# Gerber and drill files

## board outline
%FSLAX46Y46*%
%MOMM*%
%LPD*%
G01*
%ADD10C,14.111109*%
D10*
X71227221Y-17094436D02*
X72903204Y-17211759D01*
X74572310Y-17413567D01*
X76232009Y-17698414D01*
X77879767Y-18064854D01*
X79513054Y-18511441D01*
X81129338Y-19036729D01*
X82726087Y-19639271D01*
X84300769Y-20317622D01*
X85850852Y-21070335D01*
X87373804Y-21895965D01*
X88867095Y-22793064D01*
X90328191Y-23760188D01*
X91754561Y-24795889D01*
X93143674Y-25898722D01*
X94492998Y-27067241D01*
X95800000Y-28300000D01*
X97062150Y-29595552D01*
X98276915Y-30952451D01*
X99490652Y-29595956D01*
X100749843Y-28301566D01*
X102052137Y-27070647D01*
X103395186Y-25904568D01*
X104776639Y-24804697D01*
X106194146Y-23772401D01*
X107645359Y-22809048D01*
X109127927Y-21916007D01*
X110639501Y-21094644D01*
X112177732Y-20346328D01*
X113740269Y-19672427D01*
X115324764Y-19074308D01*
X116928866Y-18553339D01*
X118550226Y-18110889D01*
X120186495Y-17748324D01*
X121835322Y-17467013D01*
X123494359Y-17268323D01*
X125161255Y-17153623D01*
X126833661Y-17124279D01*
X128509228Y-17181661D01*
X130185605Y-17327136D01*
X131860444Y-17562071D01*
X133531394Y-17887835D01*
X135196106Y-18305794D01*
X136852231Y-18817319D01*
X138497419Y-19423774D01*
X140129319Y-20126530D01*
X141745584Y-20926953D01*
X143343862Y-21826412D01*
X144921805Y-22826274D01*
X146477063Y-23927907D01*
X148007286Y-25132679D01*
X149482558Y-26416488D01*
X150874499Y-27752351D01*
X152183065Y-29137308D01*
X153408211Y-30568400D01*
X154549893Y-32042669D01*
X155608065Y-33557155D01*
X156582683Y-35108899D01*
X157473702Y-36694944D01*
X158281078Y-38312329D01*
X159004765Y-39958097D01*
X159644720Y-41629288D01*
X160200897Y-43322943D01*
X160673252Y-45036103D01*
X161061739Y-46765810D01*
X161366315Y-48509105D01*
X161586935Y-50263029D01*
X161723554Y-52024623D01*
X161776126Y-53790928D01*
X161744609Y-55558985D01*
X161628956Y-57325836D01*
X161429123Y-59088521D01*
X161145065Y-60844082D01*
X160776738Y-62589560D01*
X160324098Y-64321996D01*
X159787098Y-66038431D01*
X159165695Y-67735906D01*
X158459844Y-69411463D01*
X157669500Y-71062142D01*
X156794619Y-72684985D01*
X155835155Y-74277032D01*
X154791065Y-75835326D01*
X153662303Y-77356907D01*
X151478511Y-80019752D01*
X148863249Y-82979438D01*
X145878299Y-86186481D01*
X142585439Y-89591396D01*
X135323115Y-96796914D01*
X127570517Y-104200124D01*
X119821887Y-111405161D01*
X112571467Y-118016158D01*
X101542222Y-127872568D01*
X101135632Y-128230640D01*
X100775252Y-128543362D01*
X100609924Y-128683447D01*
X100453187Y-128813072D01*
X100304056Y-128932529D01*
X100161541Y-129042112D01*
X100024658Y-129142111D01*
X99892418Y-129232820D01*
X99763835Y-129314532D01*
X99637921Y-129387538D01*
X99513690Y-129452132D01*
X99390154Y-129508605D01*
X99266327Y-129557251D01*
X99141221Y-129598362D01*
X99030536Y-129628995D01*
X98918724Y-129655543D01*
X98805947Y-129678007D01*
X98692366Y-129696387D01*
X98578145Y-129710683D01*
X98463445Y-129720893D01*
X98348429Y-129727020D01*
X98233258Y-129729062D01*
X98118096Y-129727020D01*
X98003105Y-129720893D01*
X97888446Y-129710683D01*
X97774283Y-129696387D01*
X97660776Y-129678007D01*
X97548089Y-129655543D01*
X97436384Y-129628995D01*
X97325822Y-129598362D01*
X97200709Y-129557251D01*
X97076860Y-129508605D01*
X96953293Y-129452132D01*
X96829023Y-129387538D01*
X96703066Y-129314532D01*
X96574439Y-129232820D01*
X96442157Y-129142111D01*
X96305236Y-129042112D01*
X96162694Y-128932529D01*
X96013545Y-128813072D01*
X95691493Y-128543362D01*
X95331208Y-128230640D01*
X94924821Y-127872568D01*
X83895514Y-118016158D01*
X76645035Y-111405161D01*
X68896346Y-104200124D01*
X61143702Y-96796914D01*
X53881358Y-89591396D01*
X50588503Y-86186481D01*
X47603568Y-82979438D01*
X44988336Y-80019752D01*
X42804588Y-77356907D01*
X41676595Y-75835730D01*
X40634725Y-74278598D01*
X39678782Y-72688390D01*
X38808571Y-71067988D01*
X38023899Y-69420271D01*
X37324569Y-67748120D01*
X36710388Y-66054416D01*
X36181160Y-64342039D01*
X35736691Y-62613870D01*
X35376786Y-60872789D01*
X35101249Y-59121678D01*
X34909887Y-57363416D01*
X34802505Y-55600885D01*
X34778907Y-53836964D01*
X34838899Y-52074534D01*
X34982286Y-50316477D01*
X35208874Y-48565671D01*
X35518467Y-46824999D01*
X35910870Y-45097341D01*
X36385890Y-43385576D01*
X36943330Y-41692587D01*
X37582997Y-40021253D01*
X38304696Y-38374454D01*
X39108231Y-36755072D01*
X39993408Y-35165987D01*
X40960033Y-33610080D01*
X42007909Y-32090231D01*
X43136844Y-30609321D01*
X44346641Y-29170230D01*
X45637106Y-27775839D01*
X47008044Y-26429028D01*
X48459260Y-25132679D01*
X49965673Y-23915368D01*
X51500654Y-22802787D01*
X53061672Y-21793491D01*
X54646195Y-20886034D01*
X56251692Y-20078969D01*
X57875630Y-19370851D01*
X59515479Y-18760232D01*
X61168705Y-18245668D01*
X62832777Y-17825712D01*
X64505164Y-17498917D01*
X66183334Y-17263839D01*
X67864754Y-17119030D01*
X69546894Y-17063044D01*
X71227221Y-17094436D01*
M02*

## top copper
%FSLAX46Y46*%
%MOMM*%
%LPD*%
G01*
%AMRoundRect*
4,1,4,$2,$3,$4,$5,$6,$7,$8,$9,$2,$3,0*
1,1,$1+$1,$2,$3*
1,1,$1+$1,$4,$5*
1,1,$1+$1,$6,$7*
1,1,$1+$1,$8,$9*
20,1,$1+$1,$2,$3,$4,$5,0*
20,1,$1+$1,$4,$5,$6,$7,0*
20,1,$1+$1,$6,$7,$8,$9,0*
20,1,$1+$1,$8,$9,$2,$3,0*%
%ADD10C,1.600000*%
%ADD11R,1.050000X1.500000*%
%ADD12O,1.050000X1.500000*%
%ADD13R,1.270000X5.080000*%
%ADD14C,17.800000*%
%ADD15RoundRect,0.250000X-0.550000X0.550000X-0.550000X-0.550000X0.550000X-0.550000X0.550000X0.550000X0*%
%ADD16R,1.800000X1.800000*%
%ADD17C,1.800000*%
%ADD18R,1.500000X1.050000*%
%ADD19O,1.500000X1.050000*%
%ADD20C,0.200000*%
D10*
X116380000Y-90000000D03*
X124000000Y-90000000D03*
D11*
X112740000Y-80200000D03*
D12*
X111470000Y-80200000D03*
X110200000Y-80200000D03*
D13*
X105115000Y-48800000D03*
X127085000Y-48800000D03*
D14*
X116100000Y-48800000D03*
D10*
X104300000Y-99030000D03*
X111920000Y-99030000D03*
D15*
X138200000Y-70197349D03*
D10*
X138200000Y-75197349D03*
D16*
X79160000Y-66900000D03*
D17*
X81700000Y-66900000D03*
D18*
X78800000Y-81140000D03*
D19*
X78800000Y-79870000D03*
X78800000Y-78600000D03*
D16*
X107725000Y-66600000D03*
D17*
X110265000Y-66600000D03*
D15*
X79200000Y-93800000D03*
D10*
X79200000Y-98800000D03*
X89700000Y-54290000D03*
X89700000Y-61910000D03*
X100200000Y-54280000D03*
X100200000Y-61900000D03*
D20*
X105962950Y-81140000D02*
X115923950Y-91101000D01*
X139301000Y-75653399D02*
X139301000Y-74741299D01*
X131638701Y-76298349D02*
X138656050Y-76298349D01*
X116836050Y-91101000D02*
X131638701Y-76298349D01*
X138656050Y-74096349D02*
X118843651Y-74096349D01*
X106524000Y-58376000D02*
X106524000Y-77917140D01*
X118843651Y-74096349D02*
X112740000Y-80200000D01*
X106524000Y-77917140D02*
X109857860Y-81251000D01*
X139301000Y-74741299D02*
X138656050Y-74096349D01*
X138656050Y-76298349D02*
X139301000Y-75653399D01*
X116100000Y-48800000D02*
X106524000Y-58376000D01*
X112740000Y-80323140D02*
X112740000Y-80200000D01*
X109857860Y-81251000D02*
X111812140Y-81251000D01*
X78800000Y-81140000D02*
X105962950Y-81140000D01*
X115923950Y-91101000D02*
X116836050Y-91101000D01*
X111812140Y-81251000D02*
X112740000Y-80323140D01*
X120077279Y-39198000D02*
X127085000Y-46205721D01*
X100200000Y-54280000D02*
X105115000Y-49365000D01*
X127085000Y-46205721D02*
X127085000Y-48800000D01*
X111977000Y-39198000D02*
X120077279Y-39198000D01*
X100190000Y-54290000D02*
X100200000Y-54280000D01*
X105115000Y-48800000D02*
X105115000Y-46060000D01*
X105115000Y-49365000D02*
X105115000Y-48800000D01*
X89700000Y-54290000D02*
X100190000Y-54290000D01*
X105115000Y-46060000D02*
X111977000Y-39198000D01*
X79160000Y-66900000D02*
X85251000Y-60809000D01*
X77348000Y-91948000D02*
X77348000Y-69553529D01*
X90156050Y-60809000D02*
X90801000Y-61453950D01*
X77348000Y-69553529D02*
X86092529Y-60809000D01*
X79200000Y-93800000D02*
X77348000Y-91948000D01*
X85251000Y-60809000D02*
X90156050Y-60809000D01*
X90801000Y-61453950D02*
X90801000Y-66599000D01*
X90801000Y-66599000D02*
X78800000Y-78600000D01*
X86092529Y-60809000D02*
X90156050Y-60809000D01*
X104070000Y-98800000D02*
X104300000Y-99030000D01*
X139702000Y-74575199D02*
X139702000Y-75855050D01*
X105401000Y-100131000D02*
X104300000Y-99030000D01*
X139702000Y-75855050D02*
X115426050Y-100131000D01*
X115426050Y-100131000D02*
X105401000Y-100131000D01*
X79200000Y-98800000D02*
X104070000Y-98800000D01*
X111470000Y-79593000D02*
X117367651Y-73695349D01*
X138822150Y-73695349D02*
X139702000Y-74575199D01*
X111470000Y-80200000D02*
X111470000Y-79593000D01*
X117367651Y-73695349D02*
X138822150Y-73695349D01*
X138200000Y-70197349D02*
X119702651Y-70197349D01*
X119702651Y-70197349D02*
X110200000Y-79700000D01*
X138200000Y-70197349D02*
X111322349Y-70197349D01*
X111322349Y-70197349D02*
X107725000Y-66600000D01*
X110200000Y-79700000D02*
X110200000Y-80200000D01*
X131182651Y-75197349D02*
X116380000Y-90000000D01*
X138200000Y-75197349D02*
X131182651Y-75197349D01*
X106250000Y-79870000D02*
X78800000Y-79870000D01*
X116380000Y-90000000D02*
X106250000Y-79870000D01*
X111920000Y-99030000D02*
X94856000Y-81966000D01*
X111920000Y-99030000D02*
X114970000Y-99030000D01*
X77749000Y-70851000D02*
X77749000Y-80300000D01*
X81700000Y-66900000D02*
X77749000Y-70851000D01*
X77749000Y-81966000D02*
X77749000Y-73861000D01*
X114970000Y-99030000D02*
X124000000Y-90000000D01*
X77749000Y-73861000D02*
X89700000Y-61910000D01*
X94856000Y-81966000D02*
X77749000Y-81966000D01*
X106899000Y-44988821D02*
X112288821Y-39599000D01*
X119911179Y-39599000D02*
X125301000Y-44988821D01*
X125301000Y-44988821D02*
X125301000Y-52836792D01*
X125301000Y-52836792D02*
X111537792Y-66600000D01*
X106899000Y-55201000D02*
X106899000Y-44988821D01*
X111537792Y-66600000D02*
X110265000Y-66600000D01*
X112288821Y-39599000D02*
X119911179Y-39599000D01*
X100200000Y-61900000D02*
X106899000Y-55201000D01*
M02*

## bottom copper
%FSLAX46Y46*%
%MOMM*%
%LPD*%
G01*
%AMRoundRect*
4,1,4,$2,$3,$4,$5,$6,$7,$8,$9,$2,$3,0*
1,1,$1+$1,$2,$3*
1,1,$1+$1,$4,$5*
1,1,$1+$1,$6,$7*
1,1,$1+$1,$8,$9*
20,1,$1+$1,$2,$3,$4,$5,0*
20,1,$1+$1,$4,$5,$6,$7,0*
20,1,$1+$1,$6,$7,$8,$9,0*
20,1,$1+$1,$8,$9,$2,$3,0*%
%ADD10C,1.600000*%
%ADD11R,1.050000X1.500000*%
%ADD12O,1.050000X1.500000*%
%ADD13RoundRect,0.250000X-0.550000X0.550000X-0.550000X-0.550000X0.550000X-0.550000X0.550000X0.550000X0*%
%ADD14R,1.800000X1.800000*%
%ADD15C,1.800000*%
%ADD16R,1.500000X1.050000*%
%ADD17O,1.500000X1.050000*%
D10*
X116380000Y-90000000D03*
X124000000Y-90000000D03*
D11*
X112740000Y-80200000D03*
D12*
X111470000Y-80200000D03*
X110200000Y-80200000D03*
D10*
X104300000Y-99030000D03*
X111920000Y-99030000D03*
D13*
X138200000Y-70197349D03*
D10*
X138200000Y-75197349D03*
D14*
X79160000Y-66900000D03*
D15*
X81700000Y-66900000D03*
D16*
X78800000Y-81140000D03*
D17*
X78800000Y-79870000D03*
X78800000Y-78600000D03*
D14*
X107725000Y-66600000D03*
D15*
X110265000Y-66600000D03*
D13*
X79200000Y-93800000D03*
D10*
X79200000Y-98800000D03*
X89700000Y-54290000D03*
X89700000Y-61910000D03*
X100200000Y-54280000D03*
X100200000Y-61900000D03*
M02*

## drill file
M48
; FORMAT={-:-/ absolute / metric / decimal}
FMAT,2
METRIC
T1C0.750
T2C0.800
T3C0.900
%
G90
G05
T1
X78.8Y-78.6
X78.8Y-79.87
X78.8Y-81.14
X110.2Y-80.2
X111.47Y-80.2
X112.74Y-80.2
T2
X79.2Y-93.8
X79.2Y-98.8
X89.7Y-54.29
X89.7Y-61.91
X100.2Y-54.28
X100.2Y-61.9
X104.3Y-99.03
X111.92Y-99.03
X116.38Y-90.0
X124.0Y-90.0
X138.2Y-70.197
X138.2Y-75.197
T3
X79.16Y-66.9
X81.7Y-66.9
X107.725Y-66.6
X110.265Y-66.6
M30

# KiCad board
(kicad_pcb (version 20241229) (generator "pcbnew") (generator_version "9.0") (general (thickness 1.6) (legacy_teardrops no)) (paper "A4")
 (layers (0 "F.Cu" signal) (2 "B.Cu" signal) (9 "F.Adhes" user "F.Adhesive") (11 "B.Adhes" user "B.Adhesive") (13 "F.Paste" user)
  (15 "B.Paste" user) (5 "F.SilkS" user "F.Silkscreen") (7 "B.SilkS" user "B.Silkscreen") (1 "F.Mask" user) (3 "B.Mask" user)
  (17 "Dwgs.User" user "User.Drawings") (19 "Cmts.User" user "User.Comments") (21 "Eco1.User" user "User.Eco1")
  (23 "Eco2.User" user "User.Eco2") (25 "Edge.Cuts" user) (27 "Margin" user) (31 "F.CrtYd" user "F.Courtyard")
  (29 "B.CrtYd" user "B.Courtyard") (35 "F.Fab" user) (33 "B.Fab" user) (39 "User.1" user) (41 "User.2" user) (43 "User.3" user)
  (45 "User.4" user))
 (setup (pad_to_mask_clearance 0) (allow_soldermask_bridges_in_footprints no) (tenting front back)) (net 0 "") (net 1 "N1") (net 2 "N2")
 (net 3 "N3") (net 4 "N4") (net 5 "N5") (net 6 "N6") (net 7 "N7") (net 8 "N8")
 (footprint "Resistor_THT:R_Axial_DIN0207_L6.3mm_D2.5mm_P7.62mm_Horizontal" (layer "F.Cu") (at 116.38 90)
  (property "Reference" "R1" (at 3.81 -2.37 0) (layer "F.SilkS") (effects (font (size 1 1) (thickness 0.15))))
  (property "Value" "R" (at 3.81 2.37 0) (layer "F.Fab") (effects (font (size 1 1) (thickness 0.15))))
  (pad "1" thru_hole circle (at 0 0) (size 1.6 1.6) (drill 0.8) (layers "*.Cu" "*.Mask") (remove_unused_layers no) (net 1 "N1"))
  (pad "2" thru_hole circle (at 7.62 0) (size 1.6 1.6) (drill 0.8) (layers "*.Cu" "*.Mask") (remove_unused_layers no) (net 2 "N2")))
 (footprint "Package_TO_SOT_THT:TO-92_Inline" (layer "F.Cu") (at 112.74 80.2 180)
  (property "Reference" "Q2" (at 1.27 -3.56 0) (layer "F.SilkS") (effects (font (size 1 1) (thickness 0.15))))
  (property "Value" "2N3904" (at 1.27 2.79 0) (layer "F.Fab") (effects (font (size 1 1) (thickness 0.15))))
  (pad "1" thru_hole rect (at 0 0 180) (size 1.05 1.5) (drill 0.75) (layers "*.Cu" "*.Mask") (remove_unused_layers no) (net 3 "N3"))
  (pad "2" thru_hole oval (at 1.27 0 180) (size 1.05 1.5) (drill 0.75) (layers "*.Cu" "*.Mask") (remove_unused_layers no) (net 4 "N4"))
  (pad "3" thru_hole oval (at 2.54 0 180) (size 1.05 1.5) (drill 0.75) (layers "*.Cu" "*.Mask") (remove_unused_layers no) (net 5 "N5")))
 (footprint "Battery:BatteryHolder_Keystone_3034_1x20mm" (layer "F.Cu") (at 116.1 48.8)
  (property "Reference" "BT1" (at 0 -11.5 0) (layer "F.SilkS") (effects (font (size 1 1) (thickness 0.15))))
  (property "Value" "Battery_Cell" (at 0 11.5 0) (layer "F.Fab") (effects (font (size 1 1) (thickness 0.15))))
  (pad "1" smd rect (at -10.985 0) (size 1.27 5.08) (layers "F.Cu" "F.Mask" "F.Paste") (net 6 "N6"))
  (pad "1" smd rect (at 10.985 0) (size 1.27 5.08) (layers "F.Cu" "F.Mask" "F.Paste") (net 6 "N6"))
  (pad "2" smd circle (at 0 0) (size 17.8 17.8) (layers "F.Cu" "F.Mask") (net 3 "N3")))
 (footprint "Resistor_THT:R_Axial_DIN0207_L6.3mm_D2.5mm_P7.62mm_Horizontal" (layer "F.Cu") (at 104.3 99.03)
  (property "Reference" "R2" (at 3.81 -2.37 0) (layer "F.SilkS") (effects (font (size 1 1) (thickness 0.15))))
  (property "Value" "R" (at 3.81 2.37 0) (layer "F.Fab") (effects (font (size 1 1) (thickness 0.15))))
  (pad "1" thru_hole circle (at 0 0) (size 1.6 1.6) (drill 0.8) (layers "*.Cu" "*.Mask") (remove_unused_layers no) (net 4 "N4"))
  (pad "2" thru_hole circle (at 7.62 0) (size 1.6 1.6) (drill 0.8) (layers "*.Cu" "*.Mask") (remove_unused_layers no) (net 2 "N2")))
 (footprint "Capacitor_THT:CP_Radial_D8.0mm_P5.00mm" (layer "F.Cu") (at 138.2 70.197349 -90)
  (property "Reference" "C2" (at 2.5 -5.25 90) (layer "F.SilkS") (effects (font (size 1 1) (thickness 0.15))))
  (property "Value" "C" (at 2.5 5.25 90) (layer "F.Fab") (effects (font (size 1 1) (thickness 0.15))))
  (pad "1" thru_hole roundrect (at 0 0 270) (size 1.6 1.6) (drill 0.8) (layers "*.Cu" "*.Mask") (remove_unused_layers no)
   (roundrect_rratio 0.15625) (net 5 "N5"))
  (pad "2" thru_hole circle (at 5 0 270) (size 1.6 1.6) (drill 0.8) (layers "*.Cu" "*.Mask") (remove_unused_layers no) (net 1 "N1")))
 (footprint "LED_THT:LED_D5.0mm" (layer "F.Cu") (at 79.16 66.9)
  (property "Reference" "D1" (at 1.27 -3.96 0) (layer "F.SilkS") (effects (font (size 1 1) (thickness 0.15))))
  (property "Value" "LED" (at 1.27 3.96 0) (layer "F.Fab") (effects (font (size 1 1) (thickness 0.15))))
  (pad "1" thru_hole rect (at 0 0) (size 1.8 1.8) (drill 0.9) (layers "*.Cu" "*.Mask") (remove_unused_layers no) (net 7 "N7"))
  (pad "2" thru_hole circle (at 2.54 0) (size 1.8 1.8) (drill 0.9) (layers "*.Cu" "*.Mask") (remove_unused_layers no) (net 2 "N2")))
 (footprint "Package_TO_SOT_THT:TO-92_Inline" (layer "F.Cu") (at 78.8 81.14 90)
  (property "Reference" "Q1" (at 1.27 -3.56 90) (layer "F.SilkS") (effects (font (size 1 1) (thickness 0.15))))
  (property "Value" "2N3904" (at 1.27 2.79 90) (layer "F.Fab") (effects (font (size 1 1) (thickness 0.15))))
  (pad "1" thru_hole rect (at 0 0 90) (size 1.05 1.5) (drill 0.75) (layers "*.Cu" "*.Mask") (remove_unused_layers no) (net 3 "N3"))
  (pad "2" thru_hole oval (at 1.27 0 90) (size 1.05 1.5) (drill 0.75) (layers "*.Cu" "*.Mask") (remove_unused_layers no) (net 1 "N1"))
  (pad "3" thru_hole oval (at 2.54 0 90) (size 1.05 1.5) (drill 0.75) (layers "*.Cu" "*.Mask") (remove_unused_layers no) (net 7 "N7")))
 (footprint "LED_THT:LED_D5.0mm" (layer "F.Cu") (at 107.725 66.6)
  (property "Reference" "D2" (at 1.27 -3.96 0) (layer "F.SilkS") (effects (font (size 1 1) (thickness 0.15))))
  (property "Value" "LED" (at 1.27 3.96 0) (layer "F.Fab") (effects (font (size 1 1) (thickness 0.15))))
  (pad "1" thru_hole rect (at 0 0) (size 1.8 1.8) (drill 0.9) (layers "*.Cu" "*.Mask") (remove_unused_layers no) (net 5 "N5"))
  (pad "2" thru_hole circle (at 2.54 0) (size 1.8 1.8) (drill 0.9) (layers "*.Cu" "*.Mask") (remove_unused_layers no) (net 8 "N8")))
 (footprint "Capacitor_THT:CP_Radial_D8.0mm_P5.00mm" (layer "F.Cu") (at 79.2 93.8 -90)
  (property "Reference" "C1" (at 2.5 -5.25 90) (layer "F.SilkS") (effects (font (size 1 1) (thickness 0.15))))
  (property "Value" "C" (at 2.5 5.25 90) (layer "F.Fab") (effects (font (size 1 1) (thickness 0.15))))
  (pad "1" thru_hole roundrect (at 0 0 270) (size 1.6 1.6) (drill 0.8) (layers "*.Cu" "*.Mask") (remove_unused_layers no)
   (roundrect_rratio 0.15625) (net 7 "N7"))
  (pad "2" thru_hole circle (at 5 0 270) (size 1.6 1.6) (drill 0.8) (layers "*.Cu" "*.Mask") (remove_unused_layers no) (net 4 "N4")))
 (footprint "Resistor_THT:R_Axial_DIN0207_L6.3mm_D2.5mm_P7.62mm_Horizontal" (layer "F.Cu") (at 89.7 54.29 -90)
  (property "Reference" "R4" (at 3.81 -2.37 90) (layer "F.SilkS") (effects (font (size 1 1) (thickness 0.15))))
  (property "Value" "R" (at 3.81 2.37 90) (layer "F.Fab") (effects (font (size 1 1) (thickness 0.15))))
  (pad "1" thru_hole circle (at 0 0 270) (size 1.6 1.6) (drill 0.8) (layers "*.Cu" "*.Mask") (remove_unused_layers no) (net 6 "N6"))
  (pad "2" thru_hole circle (at 7.62 0 270) (size 1.6 1.6) (drill 0.8) (layers "*.Cu" "*.Mask") (remove_unused_layers no) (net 2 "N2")))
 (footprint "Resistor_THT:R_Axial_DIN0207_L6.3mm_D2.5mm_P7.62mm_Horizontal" (layer "F.Cu") (at 100.2 54.28 -90)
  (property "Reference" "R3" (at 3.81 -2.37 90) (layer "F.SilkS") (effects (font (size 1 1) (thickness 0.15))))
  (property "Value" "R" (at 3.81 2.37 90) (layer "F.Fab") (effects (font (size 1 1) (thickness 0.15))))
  (pad "1" thru_hole circle (at 0 0 270) (size 1.6 1.6) (drill 0.8) (layers "*.Cu" "*.Mask") (remove_unused_layers no) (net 6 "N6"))
  (pad "2" thru_hole circle (at 7.62 0 270) (size 1.6 1.6) (drill 0.8) (layers "*.Cu" "*.Mask") (remove_unused_layers no) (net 8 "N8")))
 (gr_poly
  (pts (xy 71.227221 17.094436) (xy 72.903204 17.211759) (xy 74.57231 17.413567) (xy 76.232009 17.698414) (xy 77.879767 18.064854)
   (xy 79.513054 18.511441) (xy 81.129338 19.036729) (xy 82.726087 19.639271) (xy 84.300769 20.317622) (xy 85.850852 21.070335)
   (xy 87.373804 21.895965) (xy 88.867095 22.793064) (xy 90.328191 23.760188) (xy 91.754561 24.795889) (xy 93.143674 25.898722)
   (xy 94.492998 27.067241) (xy 95.8 28.3) (xy 97.06215 29.595552) (xy 98.276915 30.952451) (xy 99.490652 29.595956)
   (xy 100.749843 28.301566) (xy 102.052137 27.070647) (xy 103.395186 25.904568) (xy 104.776639 24.804697) (xy 106.194146 23.772401)
   (xy 107.645359 22.809048) (xy 109.127927 21.916007) (xy 110.639501 21.094644) (xy 112.177732 20.346328) (xy 113.740269 19.672427)
   (xy 115.324764 19.074308) (xy 116.928866 18.553339) (xy 118.550226 18.110889) (xy 120.186495 17.748324) (xy 121.835322 17.467013)
   (xy 123.494359 17.268323) (xy 125.161255 17.153623) (xy 126.833661 17.124279) (xy 128.509228 17.181661) (xy 130.185605 17.327136)
   (xy 131.860444 17.562071) (xy 133.531394 17.887835) (xy 135.196106 18.305794) (xy 136.852231 18.817319) (xy 138.497419 19.423774)
   (xy 140.129319 20.12653) (xy 141.745584 20.926953) (xy 143.343862 21.826412) (xy 144.921805 22.826274) (xy 146.477063 23.927907)
   (xy 148.007286 25.132679) (xy 149.482558 26.416488) (xy 150.874499 27.752351) (xy 152.183065 29.137308) (xy 153.408211 30.5684)
   (xy 154.549893 32.042669) (xy 155.608065 33.557155) (xy 156.582683 35.108899) (xy 157.473702 36.694944) (xy 158.281078 38.312329)
   (xy 159.004765 39.958097) (xy 159.64472 41.629288) (xy 160.200897 43.322943) (xy 160.673252 45.036103) (xy 161.061739 46.76581)
   (xy 161.366315 48.509105) (xy 161.586935 50.263029) (xy 161.723554 52.024623) (xy 161.776126 53.790928) (xy 161.744609 55.558985)
   (xy 161.628956 57.325836) (xy 161.429123 59.088521) (xy 161.145065 60.844082) (xy 160.776738 62.58956) (xy 160.324098 64.321996)
   (xy 159.787098 66.038431) (xy 159.165695 67.735906) (xy 158.459844 69.411463) (xy 157.6695 71.062142) (xy 156.794619 72.684985)
   (xy 155.835155 74.277032) (xy 154.791065 75.835326) (xy 153.662303 77.356907) (xy 151.478511 80.019752) (xy 148.863249 82.979438)
   (xy 145.878299 86.186481) (xy 142.585439 89.591396) (xy 135.323115 96.796914) (xy 127.570517 104.200124) (xy 119.821887 111.405161)
   (xy 112.571467 118.016158) (xy 101.542222 127.872568) (xy 101.135632 128.23064) (xy 100.775252 128.543362) (xy 100.609924 128.683447)
   (xy 100.453187 128.813072) (xy 100.304056 128.932529) (xy 100.161541 129.042112) (xy 100.024658 129.142111) (xy 99.892418 129.23282)
   (xy 99.763835 129.314532) (xy 99.637921 129.387538) (xy 99.51369 129.452132) (xy 99.390154 129.508605) (xy 99.266327 129.557251)
   (xy 99.141221 129.598362) (xy 99.030536 129.628995) (xy 98.918724 129.655543) (xy 98.805947 129.678007) (xy 98.692366 129.696387)
   (xy 98.578145 129.710683) (xy 98.463445 129.720893) (xy 98.348429 129.72702) (xy 98.233258 129.729062) (xy 98.118096 129.72702)
   (xy 98.003105 129.720893) (xy 97.888446 129.710683) (xy 97.774283 129.696387) (xy 97.660776 129.678007) (xy 97.548089 129.655543)
   (xy 97.436384 129.628995) (xy 97.325822 129.598362) (xy 97.200709 129.557251) (xy 97.07686 129.508605) (xy 96.953293 129.452132)
   (xy 96.829023 129.387538) (xy 96.703066 129.314532) (xy 96.574439 129.23282) (xy 96.442157 129.142111) (xy 96.305236 129.042112)
   (xy 96.162694 128.932529) (xy 96.013545 128.813072) (xy 95.691493 128.543362) (xy 95.331208 128.23064) (xy 94.924821 127.872568)
   (xy 83.895514 118.016158) (xy 76.645035 111.405161) (xy 68.896346 104.200124) (xy 61.143702 96.796914) (xy 53.881358 89.591396)
   (xy 50.588503 86.186481) (xy 47.603568 82.979438) (xy 44.988336 80.019752) (xy 42.804588 77.356907) (xy 41.676595 75.83573)
   (xy 40.634725 74.278598) (xy 39.678782 72.68839) (xy 38.808571 71.067988) (xy 38.023899 69.420271) (xy 37.324569 67.74812)
   (xy 36.710388 66.054416) (xy 36.18116 64.342039) (xy 35.736691 62.61387) (xy 35.376786 60.872789) (xy 35.101249 59.121678)
   (xy 34.909887 57.363416) (xy 34.802505 55.600885) (xy 34.778907 53.836964) (xy 34.838899 52.074534) (xy 34.982286 50.316477)
   (xy 35.208874 48.565671) (xy 35.518467 46.824999) (xy 35.91087 45.097341) (xy 36.38589 43.385576) (xy 36.94333 41.692587)
   (xy 37.582997 40.021253) (xy 38.304696 38.374454) (xy 39.108231 36.755072) (xy 39.993408 35.165987) (xy 40.960033 33.61008)
   (xy 42.007909 32.090231) (xy 43.136844 30.609321) (xy 44.346641 29.17023) (xy 45.637106 27.775839) (xy 47.008044 26.429028)
   (xy 48.45926 25.132679) (xy 49.965673 23.915368) (xy 51.500654 22.802787) (xy 53.061672 21.793491) (xy 54.646195 20.886034)
   (xy 56.251692 20.078969) (xy 57.87563 19.370851) (xy 59.515479 18.760232) (xy 61.168705 18.245668) (xy 62.832777 17.825712)
   (xy 64.505164 17.498917) (xy 66.183334 17.263839) (xy 67.864754 17.11903) (xy 69.546894 17.063044))
  (stroke (width 14.111109) (type solid)) (fill no) (layer "Edge.Cuts"))
 (segment (start 105.96295 81.14) (end 115.92395 91.101) (width 0.2) (layer "F.Cu") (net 3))
 (segment (start 139.301 75.653399) (end 139.301 74.741299) (width 0.2) (layer "F.Cu") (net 3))
 (segment (start 131.638701 76.298349) (end 138.65605 76.298349) (width 0.2) (layer "F.Cu") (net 3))
 (segment (start 116.83605 91.101) (end 131.638701 76.298349) (width 0.2) (layer "F.Cu") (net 3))
 (segment (start 138.65605 74.096349) (end 118.843651 74.096349) (width 0.2) (layer "F.Cu") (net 3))
 (segment (start 106.524 58.376) (end 106.524 77.91714) (width 0.2) (layer "F.Cu") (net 3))
 (segment (start 118.843651 74.096349) (end 112.74 80.2) (width 0.2) (layer "F.Cu") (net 3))
 (segment (start 106.524 77.91714) (end 109.85786 81.251) (width 0.2) (layer "F.Cu") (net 3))
 (segment (start 139.301 74.741299) (end 138.65605 74.096349) (width 0.2) (layer "F.Cu") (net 3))
 (segment (start 138.65605 76.298349) (end 139.301 75.653399) (width 0.2) (layer "F.Cu") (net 3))
 (segment (start 116.1 48.8) (end 106.524 58.376) (width 0.2) (layer "F.Cu") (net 3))
 (segment (start 112.74 80.32314) (end 112.74 80.2) (width 0.2) (layer "F.Cu") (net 3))
 (segment (start 109.85786 81.251) (end 111.81214 81.251) (width 0.2) (layer "F.Cu") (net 3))
 (segment (start 78.8 81.14) (end 105.96295 81.14) (width 0.2) (layer "F.Cu") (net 3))
 (segment (start 115.92395 91.101) (end 116.83605 91.101) (width 0.2) (layer "F.Cu") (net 3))
 (segment (start 111.81214 81.251) (end 112.74 80.32314) (width 0.2) (layer "F.Cu") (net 3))
 (segment (start 120.077279 39.198) (end 127.085 46.205721) (width 0.2) (layer "F.Cu") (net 6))
 (segment (start 100.2 54.28) (end 105.115 49.365) (width 0.2) (layer "F.Cu") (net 6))
 (segment (start 127.085 46.205721) (end 127.085 48.8) (width 0.2) (layer "F.Cu") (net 6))
 (segment (start 111.977 39.198) (end 120.077279 39.198) (width 0.2) (layer "F.Cu") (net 6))
 (segment (start 100.19 54.29) (end 100.2 54.28) (width 0.2) (layer "F.Cu") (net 6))
 (segment (start 105.115 48.8) (end 105.115 46.06) (width 0.2) (layer "F.Cu") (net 6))
 (segment (start 105.115 49.365) (end 105.115 48.8) (width 0.2) (layer "F.Cu") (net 6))
 (segment (start 89.7 54.29) (end 100.19 54.29) (width 0.2) (layer "F.Cu") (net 6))
 (segment (start 105.115 46.06) (end 111.977 39.198) (width 0.2) (layer "F.Cu") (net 6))
 (segment (start 79.16 66.9) (end 85.251 60.809) (width 0.2) (layer "F.Cu") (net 7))
 (segment (start 77.348 91.948) (end 77.348 69.553529) (width 0.2) (layer "F.Cu") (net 7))
 (segment (start 90.15605 60.809) (end 90.801 61.45395) (width 0.2) (layer "F.Cu") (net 7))
 (segment (start 77.348 69.553529) (end 86.092529 60.809) (width 0.2) (layer "F.Cu") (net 7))
 (segment (start 79.2 93.8) (end 77.348 91.948) (width 0.2) (layer "F.Cu") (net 7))
 (segment (start 85.251 60.809) (end 90.15605 60.809) (width 0.2) (layer "F.Cu") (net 7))
 (segment (start 90.801 61.45395) (end 90.801 66.599) (width 0.2) (layer "F.Cu") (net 7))
 (segment (start 90.801 66.599) (end 78.8 78.6) (width 0.2) (layer "F.Cu") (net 7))
 (segment (start 86.092529 60.809) (end 90.15605 60.809) (width 0.2) (layer "F.Cu") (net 7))
 (segment (start 104.07 98.8) (end 104.3 99.03) (width 0.2) (layer "F.Cu") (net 4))
 (segment (start 139.702 74.575199) (end 139.702 75.85505) (width 0.2) (layer "F.Cu") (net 4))
 (segment (start 105.401 100.131) (end 104.3 99.03) (width 0.2) (layer "F.Cu") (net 4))
 (segment (start 139.702 75.85505) (end 115.42605 100.131) (width 0.2) (layer "F.Cu") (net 4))
 (segment (start 115.42605 100.131) (end 105.401 100.131) (width 0.2) (layer "F.Cu") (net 4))
 (segment (start 79.2 98.8) (end 104.07 98.8) (width 0.2) (layer "F.Cu") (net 4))
 (segment (start 111.47 79.593) (end 117.367651 73.695349) (width 0.2) (layer "F.Cu") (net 4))
 (segment (start 138.82215 73.695349) (end 139.702 74.575199) (width 0.2) (layer "F.Cu") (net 4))
 (segment (start 111.47 80.2) (end 111.47 79.593) (width 0.2) (layer "F.Cu") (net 4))
 (segment (start 117.367651 73.695349) (end 138.82215 73.695349) (width 0.2) (layer "F.Cu") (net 4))
 (segment (start 138.2 70.197349) (end 119.702651 70.197349) (width 0.2) (layer "F.Cu") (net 5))
 (segment (start 119.702651 70.197349) (end 110.2 79.7) (width 0.2) (layer "F.Cu") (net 5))
 (segment (start 138.2 70.197349) (end 111.322349 70.197349) (width 0.2) (layer "F.Cu") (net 5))
 (segment (start 111.322349 70.197349) (end 107.725 66.6) (width 0.2) (layer "F.Cu") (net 5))
 (segment (start 110.2 79.7) (end 110.2 80.2) (width 0.2) (layer "F.Cu") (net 5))
 (segment (start 131.182651 75.197349) (end 116.38 90) (width 0.2) (layer "F.Cu") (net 1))
 (segment (start 138.2 75.197349) (end 131.182651 75.197349) (width 0.2) (layer "F.Cu") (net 1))
 (segment (start 106.25 79.87) (end 78.8 79.87) (width 0.2) (layer "F.Cu") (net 1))
 (segment (start 116.38 90) (end 106.25 79.87) (width 0.2) (layer "F.Cu") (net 1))
 (segment (start 111.92 99.03) (end 94.856 81.966) (width 0.2) (layer "F.Cu") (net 2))
 (segment (start 111.92 99.03) (end 114.97 99.03) (width 0.2) (layer "F.Cu") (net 2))
 (segment (start 77.749 70.851) (end 77.749 80.3) (width 0.2) (layer "F.Cu") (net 2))
 (segment (start 81.7 66.9) (end 77.749 70.851) (width 0.2) (layer "F.Cu") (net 2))
 (segment (start 77.749 81.966) (end 77.749 73.861) (width 0.2) (layer "F.Cu") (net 2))
 (segment (start 114.97 99.03) (end 124 90) (width 0.2) (layer "F.Cu") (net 2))
 (segment (start 77.749 73.861) (end 89.7 61.91) (width 0.2) (layer "F.Cu") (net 2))
 (segment (start 94.856 81.966) (end 77.749 81.966) (width 0.2) (layer "F.Cu") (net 2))
 (segment (start 106.899 44.988821) (end 112.288821 39.599) (width 0.2) (layer "F.Cu") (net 8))
 (segment (start 119.911179 39.599) (end 125.301 44.988821) (width 0.2) (layer "F.Cu") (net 8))
 (segment (start 125.301 44.988821) (end 125.301 52.836792) (width 0.2) (layer "F.Cu") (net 8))
 (segment (start 125.301 52.836792) (end 111.537792 66.6) (width 0.2) (layer "F.Cu") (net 8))
 (segment (start 106.899 55.201) (end 106.899 44.988821) (width 0.2) (layer "F.Cu") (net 8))
 (segment (start 111.537792 66.6) (end 110.265 66.6) (width 0.2) (layer "F.Cu") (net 8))
 (segment (start 112.288821 39.599) (end 119.911179 39.599) (width 0.2) (layer "F.Cu") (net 8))
 (segment (start 100.2 61.9) (end 106.899 55.201) (width 0.2) (layer "F.Cu") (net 8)))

